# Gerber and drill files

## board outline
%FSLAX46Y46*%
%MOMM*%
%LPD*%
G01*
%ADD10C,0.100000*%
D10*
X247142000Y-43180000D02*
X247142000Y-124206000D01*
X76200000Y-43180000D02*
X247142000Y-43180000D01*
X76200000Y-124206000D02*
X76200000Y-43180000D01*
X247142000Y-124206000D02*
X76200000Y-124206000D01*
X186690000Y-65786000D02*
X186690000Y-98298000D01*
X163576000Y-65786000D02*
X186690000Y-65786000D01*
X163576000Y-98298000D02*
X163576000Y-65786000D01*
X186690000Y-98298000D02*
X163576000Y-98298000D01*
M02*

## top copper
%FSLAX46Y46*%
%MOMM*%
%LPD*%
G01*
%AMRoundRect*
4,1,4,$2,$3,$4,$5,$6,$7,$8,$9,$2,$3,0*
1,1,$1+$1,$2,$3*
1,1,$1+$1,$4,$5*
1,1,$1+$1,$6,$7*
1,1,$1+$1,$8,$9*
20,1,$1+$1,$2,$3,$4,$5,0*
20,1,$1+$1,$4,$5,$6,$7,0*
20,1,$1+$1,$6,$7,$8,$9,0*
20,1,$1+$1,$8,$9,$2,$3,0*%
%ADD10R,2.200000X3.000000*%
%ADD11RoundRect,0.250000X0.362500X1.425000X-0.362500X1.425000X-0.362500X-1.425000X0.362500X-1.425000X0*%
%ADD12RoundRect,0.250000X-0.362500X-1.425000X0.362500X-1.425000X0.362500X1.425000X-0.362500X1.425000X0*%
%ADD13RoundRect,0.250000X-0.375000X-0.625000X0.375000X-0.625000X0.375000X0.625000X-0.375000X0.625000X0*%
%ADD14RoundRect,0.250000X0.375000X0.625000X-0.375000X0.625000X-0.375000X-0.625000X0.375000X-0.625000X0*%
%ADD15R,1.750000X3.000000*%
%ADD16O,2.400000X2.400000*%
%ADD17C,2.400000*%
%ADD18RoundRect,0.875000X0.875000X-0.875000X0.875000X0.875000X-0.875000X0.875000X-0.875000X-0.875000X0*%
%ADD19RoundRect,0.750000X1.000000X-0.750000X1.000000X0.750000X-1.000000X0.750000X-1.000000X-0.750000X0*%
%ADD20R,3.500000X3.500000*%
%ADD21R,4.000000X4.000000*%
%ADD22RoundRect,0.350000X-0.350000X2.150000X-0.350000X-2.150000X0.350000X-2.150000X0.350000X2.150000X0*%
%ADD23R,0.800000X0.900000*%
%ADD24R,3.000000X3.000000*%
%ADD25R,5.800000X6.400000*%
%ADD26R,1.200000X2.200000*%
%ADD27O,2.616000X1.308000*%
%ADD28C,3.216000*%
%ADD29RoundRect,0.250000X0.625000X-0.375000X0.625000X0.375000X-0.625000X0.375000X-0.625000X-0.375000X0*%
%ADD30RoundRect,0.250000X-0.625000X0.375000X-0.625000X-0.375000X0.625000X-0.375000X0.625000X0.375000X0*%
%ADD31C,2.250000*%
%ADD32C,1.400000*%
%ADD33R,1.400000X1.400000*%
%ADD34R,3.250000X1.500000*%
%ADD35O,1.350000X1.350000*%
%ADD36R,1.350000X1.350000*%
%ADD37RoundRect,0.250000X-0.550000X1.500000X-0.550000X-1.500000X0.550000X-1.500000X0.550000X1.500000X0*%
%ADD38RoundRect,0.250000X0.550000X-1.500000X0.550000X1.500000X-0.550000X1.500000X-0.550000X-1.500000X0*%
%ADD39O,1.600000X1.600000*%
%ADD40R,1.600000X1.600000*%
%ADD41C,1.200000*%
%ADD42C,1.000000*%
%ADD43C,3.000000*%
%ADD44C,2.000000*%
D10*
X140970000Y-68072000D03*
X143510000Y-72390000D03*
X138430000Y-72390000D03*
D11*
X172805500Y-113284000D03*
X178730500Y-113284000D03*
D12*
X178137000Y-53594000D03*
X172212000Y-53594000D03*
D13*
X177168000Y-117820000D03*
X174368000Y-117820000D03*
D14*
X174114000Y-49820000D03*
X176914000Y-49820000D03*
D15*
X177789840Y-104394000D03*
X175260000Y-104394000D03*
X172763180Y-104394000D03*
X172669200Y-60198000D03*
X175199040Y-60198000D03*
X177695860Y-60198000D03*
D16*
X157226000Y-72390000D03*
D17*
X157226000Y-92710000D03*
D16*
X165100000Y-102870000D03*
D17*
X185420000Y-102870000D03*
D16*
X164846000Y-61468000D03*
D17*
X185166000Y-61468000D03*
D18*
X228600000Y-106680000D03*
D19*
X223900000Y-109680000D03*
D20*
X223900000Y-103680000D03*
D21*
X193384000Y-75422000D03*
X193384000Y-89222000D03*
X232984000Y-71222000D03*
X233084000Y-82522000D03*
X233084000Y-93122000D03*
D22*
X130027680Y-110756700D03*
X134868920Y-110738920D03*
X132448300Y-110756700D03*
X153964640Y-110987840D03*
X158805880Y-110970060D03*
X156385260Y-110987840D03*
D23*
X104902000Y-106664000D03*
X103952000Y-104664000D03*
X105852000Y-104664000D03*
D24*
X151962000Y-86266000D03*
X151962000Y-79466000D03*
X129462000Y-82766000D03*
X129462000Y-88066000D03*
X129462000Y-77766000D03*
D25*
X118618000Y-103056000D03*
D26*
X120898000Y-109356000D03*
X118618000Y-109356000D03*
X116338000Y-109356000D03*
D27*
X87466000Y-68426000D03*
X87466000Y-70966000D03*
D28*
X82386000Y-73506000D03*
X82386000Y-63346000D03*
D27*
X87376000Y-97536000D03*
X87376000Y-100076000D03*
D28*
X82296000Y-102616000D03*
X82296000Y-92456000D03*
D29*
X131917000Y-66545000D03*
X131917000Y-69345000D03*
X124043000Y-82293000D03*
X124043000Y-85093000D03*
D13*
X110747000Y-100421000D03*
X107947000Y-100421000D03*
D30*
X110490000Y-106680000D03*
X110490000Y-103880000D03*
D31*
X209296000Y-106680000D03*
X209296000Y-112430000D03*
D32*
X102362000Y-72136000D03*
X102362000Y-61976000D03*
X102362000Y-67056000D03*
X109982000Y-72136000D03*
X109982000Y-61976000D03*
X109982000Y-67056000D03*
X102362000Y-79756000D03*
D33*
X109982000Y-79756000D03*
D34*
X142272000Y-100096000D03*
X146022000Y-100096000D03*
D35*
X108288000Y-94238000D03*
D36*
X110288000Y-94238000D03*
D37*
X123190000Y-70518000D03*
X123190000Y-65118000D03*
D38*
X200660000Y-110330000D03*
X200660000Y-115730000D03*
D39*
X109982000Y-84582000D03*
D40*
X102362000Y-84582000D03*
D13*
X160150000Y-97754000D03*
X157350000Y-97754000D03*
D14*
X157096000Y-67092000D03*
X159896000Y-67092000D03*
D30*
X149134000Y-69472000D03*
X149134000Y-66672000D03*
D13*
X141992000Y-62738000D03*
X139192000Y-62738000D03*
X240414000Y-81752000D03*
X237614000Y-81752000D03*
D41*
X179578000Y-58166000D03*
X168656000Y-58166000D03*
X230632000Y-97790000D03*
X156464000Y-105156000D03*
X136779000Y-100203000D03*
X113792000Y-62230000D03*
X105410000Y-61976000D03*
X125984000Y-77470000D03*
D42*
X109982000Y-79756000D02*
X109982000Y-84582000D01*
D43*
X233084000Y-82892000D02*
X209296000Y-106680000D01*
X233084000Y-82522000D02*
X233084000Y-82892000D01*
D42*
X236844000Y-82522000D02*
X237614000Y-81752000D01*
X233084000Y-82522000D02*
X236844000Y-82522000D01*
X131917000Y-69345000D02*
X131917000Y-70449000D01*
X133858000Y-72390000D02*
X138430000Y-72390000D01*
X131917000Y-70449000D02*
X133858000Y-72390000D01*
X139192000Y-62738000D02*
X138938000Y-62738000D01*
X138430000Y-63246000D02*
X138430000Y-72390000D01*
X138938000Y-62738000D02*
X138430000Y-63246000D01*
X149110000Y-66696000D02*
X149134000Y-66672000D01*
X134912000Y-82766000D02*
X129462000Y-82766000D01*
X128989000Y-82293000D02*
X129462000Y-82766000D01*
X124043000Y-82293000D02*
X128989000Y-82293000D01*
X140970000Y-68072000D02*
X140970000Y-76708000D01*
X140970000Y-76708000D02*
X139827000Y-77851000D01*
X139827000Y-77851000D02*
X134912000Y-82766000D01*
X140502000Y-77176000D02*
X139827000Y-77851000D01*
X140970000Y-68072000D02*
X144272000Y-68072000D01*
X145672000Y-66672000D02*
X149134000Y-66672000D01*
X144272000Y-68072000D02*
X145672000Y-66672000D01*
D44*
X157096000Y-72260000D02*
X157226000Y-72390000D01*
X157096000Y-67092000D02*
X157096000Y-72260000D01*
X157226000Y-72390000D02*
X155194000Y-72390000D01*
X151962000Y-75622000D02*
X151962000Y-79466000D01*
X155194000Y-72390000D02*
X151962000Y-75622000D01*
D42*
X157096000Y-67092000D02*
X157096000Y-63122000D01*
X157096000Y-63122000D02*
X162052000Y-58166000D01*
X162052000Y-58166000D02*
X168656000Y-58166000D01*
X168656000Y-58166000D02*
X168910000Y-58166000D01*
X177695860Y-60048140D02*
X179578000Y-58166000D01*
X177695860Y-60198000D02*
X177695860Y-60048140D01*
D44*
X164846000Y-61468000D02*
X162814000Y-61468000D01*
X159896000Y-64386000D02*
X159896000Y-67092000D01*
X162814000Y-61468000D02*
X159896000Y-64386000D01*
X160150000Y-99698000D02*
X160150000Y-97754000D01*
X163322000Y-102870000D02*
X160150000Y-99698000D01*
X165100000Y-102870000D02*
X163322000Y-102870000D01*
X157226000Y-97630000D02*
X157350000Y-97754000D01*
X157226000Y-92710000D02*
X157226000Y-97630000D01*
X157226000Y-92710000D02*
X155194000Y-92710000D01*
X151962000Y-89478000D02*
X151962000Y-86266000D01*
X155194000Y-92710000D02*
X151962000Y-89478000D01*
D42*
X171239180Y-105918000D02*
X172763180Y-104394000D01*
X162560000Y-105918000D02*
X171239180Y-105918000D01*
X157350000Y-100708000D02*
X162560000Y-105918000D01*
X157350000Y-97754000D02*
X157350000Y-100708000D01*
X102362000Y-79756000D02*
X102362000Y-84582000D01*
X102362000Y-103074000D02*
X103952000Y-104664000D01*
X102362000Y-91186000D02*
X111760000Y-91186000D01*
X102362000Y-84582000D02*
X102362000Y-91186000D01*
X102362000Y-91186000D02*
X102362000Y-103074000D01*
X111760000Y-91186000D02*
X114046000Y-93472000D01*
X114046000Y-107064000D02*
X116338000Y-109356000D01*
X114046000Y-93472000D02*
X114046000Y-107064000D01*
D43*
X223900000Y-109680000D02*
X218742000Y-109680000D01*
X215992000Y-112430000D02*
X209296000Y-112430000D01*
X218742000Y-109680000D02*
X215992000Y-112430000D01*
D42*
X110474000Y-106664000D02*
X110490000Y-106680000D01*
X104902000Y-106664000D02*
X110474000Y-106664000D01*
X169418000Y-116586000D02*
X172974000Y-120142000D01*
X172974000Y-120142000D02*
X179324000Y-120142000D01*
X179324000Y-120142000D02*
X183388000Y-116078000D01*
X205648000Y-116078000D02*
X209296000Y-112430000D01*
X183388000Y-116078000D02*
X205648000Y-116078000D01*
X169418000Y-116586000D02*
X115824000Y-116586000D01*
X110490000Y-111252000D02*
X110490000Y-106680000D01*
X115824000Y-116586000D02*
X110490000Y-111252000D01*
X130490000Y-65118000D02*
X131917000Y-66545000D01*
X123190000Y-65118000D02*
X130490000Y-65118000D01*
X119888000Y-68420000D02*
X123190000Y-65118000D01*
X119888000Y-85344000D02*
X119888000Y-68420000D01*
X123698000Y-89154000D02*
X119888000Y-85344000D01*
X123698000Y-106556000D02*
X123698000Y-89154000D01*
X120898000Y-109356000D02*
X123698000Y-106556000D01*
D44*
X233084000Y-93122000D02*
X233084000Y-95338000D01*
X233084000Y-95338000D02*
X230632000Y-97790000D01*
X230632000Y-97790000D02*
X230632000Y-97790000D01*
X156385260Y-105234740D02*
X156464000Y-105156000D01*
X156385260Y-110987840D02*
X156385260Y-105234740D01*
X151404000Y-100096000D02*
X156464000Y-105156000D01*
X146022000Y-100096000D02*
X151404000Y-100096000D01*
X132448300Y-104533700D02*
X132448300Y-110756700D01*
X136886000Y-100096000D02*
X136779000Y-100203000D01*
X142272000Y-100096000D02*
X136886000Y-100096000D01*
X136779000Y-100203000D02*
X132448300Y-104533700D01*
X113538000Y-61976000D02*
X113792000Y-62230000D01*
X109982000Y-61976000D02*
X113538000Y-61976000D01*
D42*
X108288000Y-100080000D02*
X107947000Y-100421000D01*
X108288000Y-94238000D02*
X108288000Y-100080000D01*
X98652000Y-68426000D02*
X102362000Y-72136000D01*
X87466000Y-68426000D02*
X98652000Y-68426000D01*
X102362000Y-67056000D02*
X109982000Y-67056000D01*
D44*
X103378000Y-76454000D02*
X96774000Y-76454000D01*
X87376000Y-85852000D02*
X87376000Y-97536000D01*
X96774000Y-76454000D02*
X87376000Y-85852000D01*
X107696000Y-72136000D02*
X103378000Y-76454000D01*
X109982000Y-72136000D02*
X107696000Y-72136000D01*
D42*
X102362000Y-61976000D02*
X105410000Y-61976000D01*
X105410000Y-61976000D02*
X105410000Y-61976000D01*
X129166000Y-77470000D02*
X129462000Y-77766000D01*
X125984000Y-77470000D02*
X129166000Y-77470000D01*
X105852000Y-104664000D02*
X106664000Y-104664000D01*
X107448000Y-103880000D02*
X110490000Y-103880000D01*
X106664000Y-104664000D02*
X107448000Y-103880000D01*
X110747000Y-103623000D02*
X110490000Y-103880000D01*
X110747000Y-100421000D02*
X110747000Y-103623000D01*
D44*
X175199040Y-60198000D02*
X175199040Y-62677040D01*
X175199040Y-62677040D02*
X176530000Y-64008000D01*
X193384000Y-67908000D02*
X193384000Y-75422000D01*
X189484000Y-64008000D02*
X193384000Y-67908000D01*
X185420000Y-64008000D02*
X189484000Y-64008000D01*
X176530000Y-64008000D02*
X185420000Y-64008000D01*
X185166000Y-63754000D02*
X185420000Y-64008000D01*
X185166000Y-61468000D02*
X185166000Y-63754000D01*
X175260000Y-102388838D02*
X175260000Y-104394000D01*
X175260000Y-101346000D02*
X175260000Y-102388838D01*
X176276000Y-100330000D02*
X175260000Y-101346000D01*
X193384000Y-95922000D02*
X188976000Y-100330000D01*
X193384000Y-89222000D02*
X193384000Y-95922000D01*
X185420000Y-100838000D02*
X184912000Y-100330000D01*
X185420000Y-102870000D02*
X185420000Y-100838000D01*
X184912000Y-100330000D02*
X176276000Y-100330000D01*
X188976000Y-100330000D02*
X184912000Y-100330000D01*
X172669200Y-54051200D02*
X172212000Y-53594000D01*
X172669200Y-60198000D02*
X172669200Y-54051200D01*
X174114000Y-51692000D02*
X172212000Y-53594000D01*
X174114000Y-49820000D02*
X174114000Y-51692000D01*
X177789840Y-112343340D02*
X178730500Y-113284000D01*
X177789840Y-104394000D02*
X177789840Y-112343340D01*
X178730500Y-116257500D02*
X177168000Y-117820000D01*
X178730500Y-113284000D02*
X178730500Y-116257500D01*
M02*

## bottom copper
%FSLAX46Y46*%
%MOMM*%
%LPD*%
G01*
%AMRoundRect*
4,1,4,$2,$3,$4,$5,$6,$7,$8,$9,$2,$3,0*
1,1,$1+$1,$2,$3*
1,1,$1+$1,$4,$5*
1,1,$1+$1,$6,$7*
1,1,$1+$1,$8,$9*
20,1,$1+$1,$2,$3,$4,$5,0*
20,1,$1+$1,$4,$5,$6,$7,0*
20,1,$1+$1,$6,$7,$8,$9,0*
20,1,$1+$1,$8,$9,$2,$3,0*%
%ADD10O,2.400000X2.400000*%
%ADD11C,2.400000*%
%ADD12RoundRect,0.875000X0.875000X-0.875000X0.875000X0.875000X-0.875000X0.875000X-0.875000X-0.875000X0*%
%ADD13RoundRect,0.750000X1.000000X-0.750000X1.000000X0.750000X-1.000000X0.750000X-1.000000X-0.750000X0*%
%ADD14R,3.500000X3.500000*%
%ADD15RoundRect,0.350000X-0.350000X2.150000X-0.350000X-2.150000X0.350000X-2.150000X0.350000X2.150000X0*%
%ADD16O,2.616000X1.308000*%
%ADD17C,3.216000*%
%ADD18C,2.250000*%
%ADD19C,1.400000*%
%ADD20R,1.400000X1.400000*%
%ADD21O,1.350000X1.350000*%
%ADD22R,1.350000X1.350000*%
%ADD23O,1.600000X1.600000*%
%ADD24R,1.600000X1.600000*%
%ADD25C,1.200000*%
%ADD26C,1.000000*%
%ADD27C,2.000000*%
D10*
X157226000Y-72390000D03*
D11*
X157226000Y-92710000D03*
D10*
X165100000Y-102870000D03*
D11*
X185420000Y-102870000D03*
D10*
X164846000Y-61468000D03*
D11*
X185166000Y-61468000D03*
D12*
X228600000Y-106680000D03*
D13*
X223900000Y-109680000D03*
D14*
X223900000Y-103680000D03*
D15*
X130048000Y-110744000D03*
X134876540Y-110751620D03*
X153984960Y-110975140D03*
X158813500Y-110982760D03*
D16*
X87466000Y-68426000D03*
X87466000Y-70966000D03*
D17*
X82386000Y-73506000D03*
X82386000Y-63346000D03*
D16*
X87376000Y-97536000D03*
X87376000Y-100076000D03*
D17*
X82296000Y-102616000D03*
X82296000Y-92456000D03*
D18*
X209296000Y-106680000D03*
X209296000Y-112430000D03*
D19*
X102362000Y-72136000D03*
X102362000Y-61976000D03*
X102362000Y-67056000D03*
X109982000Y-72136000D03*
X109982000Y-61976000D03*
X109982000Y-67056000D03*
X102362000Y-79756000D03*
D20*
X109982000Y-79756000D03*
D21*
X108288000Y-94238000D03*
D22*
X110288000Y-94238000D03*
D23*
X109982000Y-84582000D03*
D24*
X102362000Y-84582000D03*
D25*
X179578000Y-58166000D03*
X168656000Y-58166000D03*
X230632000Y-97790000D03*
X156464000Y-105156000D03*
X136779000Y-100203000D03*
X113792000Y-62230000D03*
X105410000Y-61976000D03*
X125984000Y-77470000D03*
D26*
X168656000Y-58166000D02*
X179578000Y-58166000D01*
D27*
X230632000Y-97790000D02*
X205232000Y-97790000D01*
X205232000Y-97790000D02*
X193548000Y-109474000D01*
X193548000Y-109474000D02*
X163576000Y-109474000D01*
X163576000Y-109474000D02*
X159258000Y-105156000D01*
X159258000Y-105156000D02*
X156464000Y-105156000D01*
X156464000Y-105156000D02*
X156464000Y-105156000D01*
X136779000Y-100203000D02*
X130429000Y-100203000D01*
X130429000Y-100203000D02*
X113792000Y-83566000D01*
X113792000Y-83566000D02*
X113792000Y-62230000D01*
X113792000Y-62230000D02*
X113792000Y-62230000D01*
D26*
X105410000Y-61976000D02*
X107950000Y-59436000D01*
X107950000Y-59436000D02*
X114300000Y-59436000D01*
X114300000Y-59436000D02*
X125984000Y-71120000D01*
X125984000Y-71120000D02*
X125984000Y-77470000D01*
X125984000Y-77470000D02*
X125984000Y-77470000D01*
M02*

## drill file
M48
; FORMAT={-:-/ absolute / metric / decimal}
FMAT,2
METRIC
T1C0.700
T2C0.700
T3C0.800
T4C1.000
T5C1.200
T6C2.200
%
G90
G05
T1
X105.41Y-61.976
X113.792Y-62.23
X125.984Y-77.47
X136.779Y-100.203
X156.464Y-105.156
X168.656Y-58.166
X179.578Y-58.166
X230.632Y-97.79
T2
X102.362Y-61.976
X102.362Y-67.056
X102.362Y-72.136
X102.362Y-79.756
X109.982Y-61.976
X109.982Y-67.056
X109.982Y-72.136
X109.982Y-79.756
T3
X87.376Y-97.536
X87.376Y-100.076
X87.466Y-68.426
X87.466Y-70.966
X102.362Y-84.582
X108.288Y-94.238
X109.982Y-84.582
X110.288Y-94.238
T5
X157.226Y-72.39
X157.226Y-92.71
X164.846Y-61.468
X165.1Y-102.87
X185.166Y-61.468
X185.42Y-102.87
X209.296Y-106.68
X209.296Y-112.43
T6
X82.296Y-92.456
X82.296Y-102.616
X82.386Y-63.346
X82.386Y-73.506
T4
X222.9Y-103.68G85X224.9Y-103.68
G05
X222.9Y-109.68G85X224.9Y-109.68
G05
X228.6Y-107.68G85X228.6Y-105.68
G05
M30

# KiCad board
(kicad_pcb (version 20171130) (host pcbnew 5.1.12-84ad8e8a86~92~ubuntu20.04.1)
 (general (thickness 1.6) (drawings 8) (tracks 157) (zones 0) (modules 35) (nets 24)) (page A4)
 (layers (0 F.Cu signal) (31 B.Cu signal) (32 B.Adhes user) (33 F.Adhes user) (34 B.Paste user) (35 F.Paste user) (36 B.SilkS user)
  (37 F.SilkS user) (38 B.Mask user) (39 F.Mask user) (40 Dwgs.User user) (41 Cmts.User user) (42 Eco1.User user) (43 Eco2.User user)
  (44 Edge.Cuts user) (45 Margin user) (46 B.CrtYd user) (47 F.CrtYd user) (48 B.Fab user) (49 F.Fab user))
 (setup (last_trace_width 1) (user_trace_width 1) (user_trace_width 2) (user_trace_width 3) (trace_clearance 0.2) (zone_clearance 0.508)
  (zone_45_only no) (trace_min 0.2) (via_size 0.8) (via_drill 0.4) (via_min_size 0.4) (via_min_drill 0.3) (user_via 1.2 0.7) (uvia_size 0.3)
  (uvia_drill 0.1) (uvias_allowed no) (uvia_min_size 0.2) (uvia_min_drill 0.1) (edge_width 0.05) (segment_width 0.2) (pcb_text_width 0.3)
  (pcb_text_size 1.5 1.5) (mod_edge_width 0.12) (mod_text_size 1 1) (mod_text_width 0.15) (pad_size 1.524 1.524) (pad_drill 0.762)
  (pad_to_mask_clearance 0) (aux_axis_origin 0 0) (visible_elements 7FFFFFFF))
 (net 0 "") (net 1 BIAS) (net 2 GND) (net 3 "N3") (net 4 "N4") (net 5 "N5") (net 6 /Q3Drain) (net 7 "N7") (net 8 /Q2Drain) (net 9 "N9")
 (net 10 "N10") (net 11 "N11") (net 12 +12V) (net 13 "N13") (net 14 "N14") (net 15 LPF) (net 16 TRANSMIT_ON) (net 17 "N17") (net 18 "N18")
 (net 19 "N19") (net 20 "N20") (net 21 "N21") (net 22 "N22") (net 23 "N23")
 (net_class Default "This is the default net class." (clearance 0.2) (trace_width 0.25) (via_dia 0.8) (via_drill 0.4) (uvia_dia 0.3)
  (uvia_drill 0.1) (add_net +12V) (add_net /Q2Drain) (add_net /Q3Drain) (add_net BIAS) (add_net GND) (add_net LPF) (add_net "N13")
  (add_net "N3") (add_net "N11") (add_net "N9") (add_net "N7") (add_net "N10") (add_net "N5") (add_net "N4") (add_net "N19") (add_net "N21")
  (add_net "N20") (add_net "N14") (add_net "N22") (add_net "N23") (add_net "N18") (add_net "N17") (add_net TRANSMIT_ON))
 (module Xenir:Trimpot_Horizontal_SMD (layer F.Cu) (at 135.636 70.358 90)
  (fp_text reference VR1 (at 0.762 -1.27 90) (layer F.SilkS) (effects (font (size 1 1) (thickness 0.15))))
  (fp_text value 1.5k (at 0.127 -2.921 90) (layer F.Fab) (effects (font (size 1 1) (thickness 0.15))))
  (pad 2 smd rect (at 2.286 5.334 90) (size 3 2.2) (layers F.Cu F.Paste F.Mask) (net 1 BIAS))
  (pad 3 smd rect (at -2.032 7.874 90) (size 3 2.2) (layers F.Cu F.Paste F.Mask) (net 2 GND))
  (pad 1 smd rect (at -2.032 2.794 90) (size 3 2.2) (layers F.Cu F.Paste F.Mask) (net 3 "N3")))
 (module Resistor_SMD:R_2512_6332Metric (layer F.Cu) (at 175.768 113.284 180)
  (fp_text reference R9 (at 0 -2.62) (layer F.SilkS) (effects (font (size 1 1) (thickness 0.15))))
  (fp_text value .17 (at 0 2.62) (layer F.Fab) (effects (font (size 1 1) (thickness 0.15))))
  (pad 2 smd roundrect (at 2.9625 0 180) (size 1.225 3.35) (layers F.Cu F.Paste F.Mask) (roundrect_rratio 0.204082) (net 2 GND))
  (pad 1 smd roundrect (at -2.9625 0 180) (size 1.225 3.35) (layers F.Cu F.Paste F.Mask) (roundrect_rratio 0.204082) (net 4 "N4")))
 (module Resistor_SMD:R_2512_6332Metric (layer F.Cu) (at 175.1745 53.594)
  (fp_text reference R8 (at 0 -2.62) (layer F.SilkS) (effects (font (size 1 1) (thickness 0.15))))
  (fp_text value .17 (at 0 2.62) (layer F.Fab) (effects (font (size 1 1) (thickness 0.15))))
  (pad 2 smd roundrect (at 2.9625 0) (size 1.225 3.35) (layers F.Cu F.Paste F.Mask) (roundrect_rratio 0.204082) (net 2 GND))
  (pad 1 smd roundrect (at -2.9625 0) (size 1.225 3.35) (layers F.Cu F.Paste F.Mask) (roundrect_rratio 0.204082) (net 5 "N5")))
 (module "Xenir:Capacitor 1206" (layer F.Cu) (at 175.768 115.57)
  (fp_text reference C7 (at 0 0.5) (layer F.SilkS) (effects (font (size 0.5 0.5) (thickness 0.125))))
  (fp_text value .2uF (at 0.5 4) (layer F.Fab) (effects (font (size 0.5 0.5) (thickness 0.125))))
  (pad 2 smd roundrect (at 1.4 2.25) (size 1.25 1.75) (layers F.Cu F.Paste F.Mask) (roundrect_rratio 0.2) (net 4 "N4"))
  (pad 1 smd roundrect (at -1.4 2.25) (size 1.25 1.75) (layers F.Cu F.Paste F.Mask) (roundrect_rratio 0.2) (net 2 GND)))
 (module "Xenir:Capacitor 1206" (layer F.Cu) (at 175.514 52.07 180)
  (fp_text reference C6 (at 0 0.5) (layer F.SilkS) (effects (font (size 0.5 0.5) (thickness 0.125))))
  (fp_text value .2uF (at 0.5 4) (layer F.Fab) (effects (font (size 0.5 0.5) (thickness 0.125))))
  (pad 2 smd roundrect (at 1.4 2.25 180) (size 1.25 1.75) (layers F.Cu F.Paste F.Mask) (roundrect_rratio 0.2) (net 5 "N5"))
  (pad 1 smd roundrect (at -1.4 2.25 180) (size 1.25 1.75) (layers F.Cu F.Paste F.Mask) (roundrect_rratio 0.2) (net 2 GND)))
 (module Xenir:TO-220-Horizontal (layer F.Cu) (at 175.45304 98.43918)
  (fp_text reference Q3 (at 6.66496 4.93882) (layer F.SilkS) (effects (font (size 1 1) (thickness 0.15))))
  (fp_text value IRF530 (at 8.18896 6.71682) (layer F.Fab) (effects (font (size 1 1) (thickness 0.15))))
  (pad 3 smd rect (at 2.3368 5.95482) (size 1.75 3) (layers F.Cu F.Paste F.Mask) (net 4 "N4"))
  (pad 2 smd rect (at -0.19304 5.95482) (size 1.75 3) (layers F.Cu F.Paste F.Mask) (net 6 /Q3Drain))
  (pad 1 smd rect (at -2.68986 5.95482) (size 1.75 3) (layers F.Cu F.Paste F.Mask) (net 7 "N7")))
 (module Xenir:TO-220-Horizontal (layer F.Cu) (at 175.006 66.15282 180)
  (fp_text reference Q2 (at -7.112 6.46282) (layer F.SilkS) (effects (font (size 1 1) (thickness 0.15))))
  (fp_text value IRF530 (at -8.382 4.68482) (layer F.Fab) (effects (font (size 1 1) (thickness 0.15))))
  (pad 3 smd rect (at 2.3368 5.95482 180) (size 1.75 3) (layers F.Cu F.Paste F.Mask) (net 5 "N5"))
  (pad 2 smd rect (at -0.19304 5.95482 180) (size 1.75 3) (layers F.Cu F.Paste F.Mask) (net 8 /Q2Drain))
  (pad 1 smd rect (at -2.68986 5.95482 180) (size 1.75 3) (layers F.Cu F.Paste F.Mask) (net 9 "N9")))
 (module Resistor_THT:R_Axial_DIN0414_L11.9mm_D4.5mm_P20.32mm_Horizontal (layer F.Cu) (at 157.226 92.71 90)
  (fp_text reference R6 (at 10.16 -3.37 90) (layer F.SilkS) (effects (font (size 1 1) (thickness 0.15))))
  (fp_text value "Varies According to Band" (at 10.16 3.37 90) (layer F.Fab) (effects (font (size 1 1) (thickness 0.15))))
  (pad 2 thru_hole oval (at 20.32 0 90) (size 2.4 2.4) (drill 1.2) (layers *.Cu *.Mask) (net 9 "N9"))
  (pad 1 thru_hole circle (at 0 0 90) (size 2.4 2.4) (drill 1.2) (layers *.Cu *.Mask) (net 7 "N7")))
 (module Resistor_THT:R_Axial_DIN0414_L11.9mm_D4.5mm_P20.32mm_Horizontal (layer F.Cu) (at 185.42 102.87 180)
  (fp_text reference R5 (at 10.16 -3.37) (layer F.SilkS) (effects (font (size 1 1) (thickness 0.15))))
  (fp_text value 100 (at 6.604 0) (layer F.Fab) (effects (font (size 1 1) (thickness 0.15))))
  (pad 2 thru_hole oval (at 20.32 0 180) (size 2.4 2.4) (drill 1.2) (layers *.Cu *.Mask) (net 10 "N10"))
  (pad 1 thru_hole circle (at 0 0 180) (size 2.4 2.4) (drill 1.2) (layers *.Cu *.Mask) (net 6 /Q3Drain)))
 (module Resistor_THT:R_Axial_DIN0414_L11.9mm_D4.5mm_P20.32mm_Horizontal (layer F.Cu) (at 185.166 61.468 180)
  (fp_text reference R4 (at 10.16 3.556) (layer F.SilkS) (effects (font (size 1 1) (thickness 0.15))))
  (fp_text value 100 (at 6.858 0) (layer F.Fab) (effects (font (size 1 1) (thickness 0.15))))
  (pad 2 thru_hole oval (at 20.32 0 180) (size 2.4 2.4) (drill 1.2) (layers *.Cu *.Mask) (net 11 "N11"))
  (pad 1 thru_hole circle (at 0 0 180) (size 2.4 2.4) (drill 1.2) (layers *.Cu *.Mask) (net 8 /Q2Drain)))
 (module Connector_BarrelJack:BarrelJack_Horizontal (layer F.Cu) (at 223.9 103.68 90)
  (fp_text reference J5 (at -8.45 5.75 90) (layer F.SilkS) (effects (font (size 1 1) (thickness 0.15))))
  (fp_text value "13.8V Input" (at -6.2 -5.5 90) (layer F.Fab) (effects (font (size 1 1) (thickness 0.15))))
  (pad 3 thru_hole roundrect (at -3 4.7 90) (size 3.5 3.5) (drill oval 3 1) (layers *.Cu *.Mask) (roundrect_rratio 0.25))
  (pad 2 thru_hole roundrect (at -6 0 90) (size 3 3.5) (drill oval 1 3) (layers *.Cu *.Mask) (roundrect_rratio 0.25) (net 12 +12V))
  (pad 1 thru_hole rect (at 0 0 90) (size 3.5 3.5) (drill oval 1 3) (layers *.Cu *.Mask) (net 2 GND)))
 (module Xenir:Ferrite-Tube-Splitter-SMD (layer F.Cu) (at 214.884 99.822 180)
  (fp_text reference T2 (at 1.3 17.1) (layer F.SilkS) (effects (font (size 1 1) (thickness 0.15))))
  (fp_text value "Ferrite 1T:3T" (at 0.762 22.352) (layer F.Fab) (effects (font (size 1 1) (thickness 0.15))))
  (pad 5 smd rect (at 21.5 24.4 180) (size 4 4) (layers F.Cu F.Paste F.Mask) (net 8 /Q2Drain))
  (pad 3 smd rect (at 21.5 10.6 180) (size 4 4) (layers F.Cu F.Paste F.Mask) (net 6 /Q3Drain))
  (pad 2 smd rect (at -18.1 28.6 180) (size 4 4) (layers F.Cu F.Paste F.Mask) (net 2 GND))
  (pad 4 smd rect (at -18.2 17.3 180) (size 4 4) (layers F.Cu F.Paste F.Mask) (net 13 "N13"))
  (pad 1 smd rect (at -18.2 6.7 180) (size 4 4) (layers F.Cu F.Paste F.Mask) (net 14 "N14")))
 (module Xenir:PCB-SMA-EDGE (layer F.Cu) (at 137.60704 110.76686 270)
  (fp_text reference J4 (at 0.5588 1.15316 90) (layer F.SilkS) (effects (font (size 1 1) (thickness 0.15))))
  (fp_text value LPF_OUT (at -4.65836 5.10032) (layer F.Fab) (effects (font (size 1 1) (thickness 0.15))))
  (pad 2 smd roundrect (at -0.02286 7.55904 270) (size 5 1.4) (layers B.Cu F.Paste F.Mask) (roundrect_rratio 0.25) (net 2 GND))
  (pad 2 smd roundrect (at -0.01524 2.7305 270) (size 5 1.4) (layers B.Cu F.Paste F.Mask) (roundrect_rratio 0.25) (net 2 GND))
  (pad 2 smd roundrect (at -0.01016 7.57936 270) (size 5 1.4) (layers F.Cu F.Paste F.Mask) (roundrect_rratio 0.25) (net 2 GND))
  (pad 2 smd roundrect (at -0.02794 2.73812 270) (size 5 1.4) (layers F.Cu F.Paste F.Mask) (roundrect_rratio 0.25) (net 2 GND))
  (pad 1 smd roundrect (at -0.01016 5.15874 270) (size 5 1.4) (layers F.Cu F.Paste F.Mask) (roundrect_rratio 0.25) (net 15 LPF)))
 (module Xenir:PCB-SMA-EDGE (layer F.Cu) (at 161.544 110.998 270)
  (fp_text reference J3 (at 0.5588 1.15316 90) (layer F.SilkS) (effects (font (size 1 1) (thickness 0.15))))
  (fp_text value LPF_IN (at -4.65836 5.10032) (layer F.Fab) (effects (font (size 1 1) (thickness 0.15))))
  (pad 2 smd roundrect (at -0.02286 7.55904 270) (size 5 1.4) (layers B.Cu F.Paste F.Mask) (roundrect_rratio 0.25) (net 2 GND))
  (pad 2 smd roundrect (at -0.01524 2.7305 270) (size 5 1.4) (layers B.Cu F.Paste F.Mask) (roundrect_rratio 0.25) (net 2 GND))
  (pad 2 smd roundrect (at -0.01016 7.57936 270) (size 5 1.4) (layers F.Cu F.Paste F.Mask) (roundrect_rratio 0.25) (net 2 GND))
  (pad 2 smd roundrect (at -0.02794 2.73812 270) (size 5 1.4) (layers F.Cu F.Paste F.Mask) (roundrect_rratio 0.25) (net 2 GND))
  (pad 1 smd roundrect (at -0.01016 5.15874 270) (size 5 1.4) (layers F.Cu F.Paste F.Mask) (roundrect_rratio 0.25) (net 14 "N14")))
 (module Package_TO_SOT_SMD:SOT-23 (layer F.Cu) (at 104.902 105.664 270)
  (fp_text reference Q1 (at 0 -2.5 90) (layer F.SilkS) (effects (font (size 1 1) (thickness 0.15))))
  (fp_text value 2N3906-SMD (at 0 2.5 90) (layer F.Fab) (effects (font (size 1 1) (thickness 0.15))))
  (pad 3 smd rect (at 1 0 270) (size 0.9 0.8) (layers F.Cu F.Paste F.Mask) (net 12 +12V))
  (pad 2 smd rect (at -1 0.95 270) (size 0.9 0.8) (layers F.Cu F.Paste F.Mask) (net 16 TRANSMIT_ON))
  (pad 1 smd rect (at -1 -0.95 270) (size 0.9 0.8) (layers F.Cu F.Paste F.Mask) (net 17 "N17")))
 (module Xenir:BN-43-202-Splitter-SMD (layer F.Cu) (at 140.462 70.866)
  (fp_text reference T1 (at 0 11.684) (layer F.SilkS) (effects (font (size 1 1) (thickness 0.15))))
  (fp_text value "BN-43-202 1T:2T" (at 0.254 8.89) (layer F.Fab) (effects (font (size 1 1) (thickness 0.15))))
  (pad 5 smd rect (at 11.5 15.4) (size 3 3) (layers F.Cu F.Paste F.Mask) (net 7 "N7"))
  (pad 3 smd rect (at 11.5 8.6) (size 3 3) (layers F.Cu F.Paste F.Mask) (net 9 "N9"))
  (pad 4 smd rect (at -11 11.9) (size 3 3) (layers F.Cu F.Paste F.Mask) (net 1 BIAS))
  (pad 2 smd rect (at -11 17.2) (size 3 3) (layers F.Cu F.Paste F.Mask) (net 2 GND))
  (pad 1 smd rect (at -11 6.9) (size 3 3) (layers F.Cu F.Paste F.Mask) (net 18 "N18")))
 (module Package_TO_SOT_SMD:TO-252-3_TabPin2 (layer F.Cu) (at 118.618 105.156 90)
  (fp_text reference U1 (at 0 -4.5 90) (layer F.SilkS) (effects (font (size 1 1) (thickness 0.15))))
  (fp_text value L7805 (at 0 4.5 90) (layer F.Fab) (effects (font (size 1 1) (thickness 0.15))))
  (pad "" smd rect (at 0.425 1.525 90) (size 3.05 2.75) (layers F.Paste))
  (pad "" smd rect (at 3.775 -1.525 90) (size 3.05 2.75) (layers F.Paste))
  (pad "" smd rect (at 0.425 -1.525 90) (size 3.05 2.75) (layers F.Paste))
  (pad "" smd rect (at 3.775 1.525 90) (size 3.05 2.75) (layers F.Paste))
  (pad 2 smd rect (at 2.1 0 90) (size 6.4 5.8) (layers F.Cu F.Mask) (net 2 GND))
  (pad 3 smd rect (at -4.2 2.28 90) (size 2.2 1.2) (layers F.Cu F.Paste F.Mask) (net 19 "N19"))
  (pad 2 smd rect (at -4.2 0 90) (size 2.2 1.2) (layers F.Cu F.Paste F.Mask) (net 2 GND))
  (pad 1 smd rect (at -4.2 -2.28 90) (size 2.2 1.2) (layers F.Cu F.Paste F.Mask) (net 16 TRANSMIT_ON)))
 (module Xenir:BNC (layer F.Cu) (at 83.566 68.326 90)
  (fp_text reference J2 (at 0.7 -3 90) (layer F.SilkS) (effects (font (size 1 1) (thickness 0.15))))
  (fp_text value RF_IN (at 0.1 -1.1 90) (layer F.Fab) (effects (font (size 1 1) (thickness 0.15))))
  (pad S thru_hole oval (at -0.1 3.9 180) (size 2.616 1.308) (drill 0.8) (layers *.Cu *.Mask) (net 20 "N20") (solder_mask_margin 0.1016))
  (pad GND thru_hole oval (at -2.64 3.9 180) (size 2.616 1.308) (drill 0.8) (layers *.Cu *.Mask) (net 2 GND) (solder_mask_margin 0.1016))
  (pad 3 thru_hole circle (at -5.18 -1.18 90) (size 3.216 3.216) (drill 2.2) (layers *.Cu *.Mask) (solder_mask_margin 0.1016))
  (pad 4 thru_hole circle (at 4.98 -1.18 90) (size 3.216 3.216) (drill 2.2) (layers *.Cu *.Mask) (solder_mask_margin 0.1016)))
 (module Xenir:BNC (layer F.Cu) (at 83.476 97.436 90)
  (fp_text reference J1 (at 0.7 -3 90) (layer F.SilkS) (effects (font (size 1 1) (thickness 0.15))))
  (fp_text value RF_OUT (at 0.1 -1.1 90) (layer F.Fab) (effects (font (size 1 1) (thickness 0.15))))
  (pad S thru_hole oval (at -0.1 3.9 180) (size 2.616 1.308) (drill 0.8) (layers *.Cu *.Mask) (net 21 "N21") (solder_mask_margin 0.1016))
  (pad GND thru_hole oval (at -2.64 3.9 180) (size 2.616 1.308) (drill 0.8) (layers *.Cu *.Mask) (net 2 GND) (solder_mask_margin 0.1016))
  (pad 3 thru_hole circle (at -5.18 -1.18 90) (size 3.216 3.216) (drill 2.2) (layers *.Cu *.Mask) (solder_mask_margin 0.1016))
  (pad 4 thru_hole circle (at 4.98 -1.18 90) (size 3.216 3.216) (drill 2.2) (layers *.Cu *.Mask) (solder_mask_margin 0.1016)))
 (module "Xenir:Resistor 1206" (layer F.Cu) (at 129.54 67.818 90)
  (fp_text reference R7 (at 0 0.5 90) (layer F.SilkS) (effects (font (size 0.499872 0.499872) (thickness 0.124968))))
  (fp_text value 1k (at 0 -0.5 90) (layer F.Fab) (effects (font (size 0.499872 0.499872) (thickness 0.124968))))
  (pad 2 smd roundrect (at 1.273 2.377 90) (size 1.25 1.75) (layers F.Cu F.Paste F.Mask) (roundrect_rratio 0.2) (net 19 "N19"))
  (pad 1 smd roundrect (at -1.527 2.377 90) (size 1.25 1.75) (layers F.Cu F.Paste F.Mask) (roundrect_rratio 0.2) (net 3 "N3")))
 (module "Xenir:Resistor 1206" (layer F.Cu) (at 121.666 83.566 90)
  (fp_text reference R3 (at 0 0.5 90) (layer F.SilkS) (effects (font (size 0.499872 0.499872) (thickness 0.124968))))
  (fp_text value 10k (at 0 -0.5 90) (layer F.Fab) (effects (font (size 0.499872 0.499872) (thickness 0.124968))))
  (pad 2 smd roundrect (at 1.273 2.377 90) (size 1.25 1.75) (layers F.Cu F.Paste F.Mask) (roundrect_rratio 0.2) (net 1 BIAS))
  (pad 1 smd roundrect (at -1.527 2.377 90) (size 1.25 1.75) (layers F.Cu F.Paste F.Mask) (roundrect_rratio 0.2) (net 2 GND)))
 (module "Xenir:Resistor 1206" (layer F.Cu) (at 109.474 98.044)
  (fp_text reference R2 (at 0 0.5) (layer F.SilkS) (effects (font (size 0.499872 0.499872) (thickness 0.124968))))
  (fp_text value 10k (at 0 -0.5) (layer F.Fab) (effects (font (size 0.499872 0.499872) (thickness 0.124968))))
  (pad 2 smd roundrect (at 1.273 2.377) (size 1.25 1.75) (layers F.Cu F.Paste F.Mask) (roundrect_rratio 0.2) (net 17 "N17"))
  (pad 1 smd roundrect (at -1.527 2.377) (size 1.25 1.75) (layers F.Cu F.Paste F.Mask) (roundrect_rratio 0.2) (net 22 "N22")))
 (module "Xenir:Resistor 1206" (layer F.Cu) (at 112.867 105.407 270)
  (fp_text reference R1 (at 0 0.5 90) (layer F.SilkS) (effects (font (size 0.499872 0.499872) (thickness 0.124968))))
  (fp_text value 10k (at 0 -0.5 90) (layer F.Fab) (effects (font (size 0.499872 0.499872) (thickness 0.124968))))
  (pad 2 smd roundrect (at 1.273 2.377 270) (size 1.25 1.75) (layers F.Cu F.Paste F.Mask) (roundrect_rratio 0.2) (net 12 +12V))
  (pad 1 smd roundrect (at -1.527 2.377 270) (size 1.25 1.75) (layers F.Cu F.Paste F.Mask) (roundrect_rratio 0.2) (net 17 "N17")))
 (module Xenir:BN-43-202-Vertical (layer F.Cu) (at 209.296 117.43 180)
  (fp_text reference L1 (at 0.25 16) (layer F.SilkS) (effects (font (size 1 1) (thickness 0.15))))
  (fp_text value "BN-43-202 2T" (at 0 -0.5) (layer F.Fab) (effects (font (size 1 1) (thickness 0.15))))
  (pad 2 thru_hole circle (at 0 10.75 180) (size 2.25 2.25) (drill 1.2) (layers *.Cu *.Mask) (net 13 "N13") (solder_mask_margin 0.1016))
  (pad 1 thru_hole circle (at 0 5 180) (size 2.25 2.25) (drill 1.2) (layers *.Cu *.Mask) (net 12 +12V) (solder_mask_margin 0.1016)))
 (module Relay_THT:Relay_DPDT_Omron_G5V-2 (layer F.Cu) (at 109.982 79.756 180)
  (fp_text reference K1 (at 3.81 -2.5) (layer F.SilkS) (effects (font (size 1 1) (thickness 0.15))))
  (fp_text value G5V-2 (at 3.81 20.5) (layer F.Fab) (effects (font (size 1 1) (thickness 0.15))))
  (pad 13 thru_hole circle (at 7.62 7.62 180) (size 1.4 1.4) (drill 0.7) (layers *.Cu *.Mask) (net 20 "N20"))
  (pad 9 thru_hole circle (at 7.62 17.78 180) (size 1.4 1.4) (drill 0.7) (layers *.Cu *.Mask) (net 18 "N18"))
  (pad 11 thru_hole circle (at 7.62 12.7 180) (size 1.4 1.4) (drill 0.7) (layers *.Cu *.Mask) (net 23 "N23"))
  (pad 4 thru_hole circle (at 0 7.62 180) (size 1.4 1.4) (drill 0.7) (layers *.Cu *.Mask) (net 21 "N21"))
  (pad 8 thru_hole circle (at 0 17.78 180) (size 1.4 1.4) (drill 0.7) (layers *.Cu *.Mask) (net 15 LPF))
  (pad 6 thru_hole circle (at 0 12.7 180) (size 1.4 1.4) (drill 0.7) (layers *.Cu *.Mask) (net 23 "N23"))
  (pad 16 thru_hole circle (at 7.62 0 180) (size 1.4 1.4) (drill 0.7) (layers *.Cu *.Mask) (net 16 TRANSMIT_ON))
  (pad 1 thru_hole rect (at 0 0 180) (size 1.4 1.4) (drill 0.7) (layers *.Cu *.Mask) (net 2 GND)))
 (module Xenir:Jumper (layer F.Cu) (at 144.272 101.346 180)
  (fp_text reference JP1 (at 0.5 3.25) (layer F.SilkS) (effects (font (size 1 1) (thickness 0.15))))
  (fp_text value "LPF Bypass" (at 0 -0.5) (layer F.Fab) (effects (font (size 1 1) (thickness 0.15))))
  (pad 2 smd rect (at 2 1.25 180) (size 3.25 1.5) (layers F.Cu F.Mask) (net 15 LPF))
  (pad 1 smd rect (at -1.75 1.25 180) (size 3.25 1.5) (layers F.Cu F.Mask) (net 14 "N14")))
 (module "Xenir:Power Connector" (layer F.Cu) (at 113.538 94.488 270)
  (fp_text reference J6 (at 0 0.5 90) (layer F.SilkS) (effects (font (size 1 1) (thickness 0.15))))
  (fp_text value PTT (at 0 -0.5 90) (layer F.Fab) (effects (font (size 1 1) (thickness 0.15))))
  (pad 2 thru_hole oval (at -0.25 5.25 270) (size 1.35 1.35) (drill 0.8) (layers *.Cu *.Mask) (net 22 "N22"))
  (pad 1 thru_hole rect (at -0.25 3.25 270) (size 1.35 1.35) (drill 0.8) (layers *.Cu *.Mask) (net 2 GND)))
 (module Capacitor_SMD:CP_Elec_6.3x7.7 (layer F.Cu) (at 123.19 67.818 270)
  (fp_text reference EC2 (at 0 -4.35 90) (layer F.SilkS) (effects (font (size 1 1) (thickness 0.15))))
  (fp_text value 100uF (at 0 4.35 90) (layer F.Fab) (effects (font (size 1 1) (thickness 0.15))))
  (pad 2 smd roundrect (at 2.7 0 270) (size 3.5 1.6) (layers F.Cu F.Paste F.Mask) (roundrect_rratio 0.15625) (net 2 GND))
  (pad 1 smd roundrect (at -2.7 0 270) (size 3.5 1.6) (layers F.Cu F.Paste F.Mask) (roundrect_rratio 0.15625) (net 19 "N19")))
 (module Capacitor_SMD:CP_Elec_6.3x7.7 (layer F.Cu) (at 200.66 113.03 90)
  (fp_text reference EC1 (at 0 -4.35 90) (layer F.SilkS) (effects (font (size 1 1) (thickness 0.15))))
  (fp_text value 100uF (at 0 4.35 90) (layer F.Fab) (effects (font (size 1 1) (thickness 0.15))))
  (pad 2 smd roundrect (at 2.7 0 90) (size 3.5 1.6) (layers F.Cu F.Paste F.Mask) (roundrect_rratio 0.15625) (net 2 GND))
  (pad 1 smd roundrect (at -2.7 0 90) (size 3.5 1.6) (layers F.Cu F.Paste F.Mask) (roundrect_rratio 0.15625) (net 12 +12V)))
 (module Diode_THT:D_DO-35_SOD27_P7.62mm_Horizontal (layer F.Cu) (at 102.362 84.582)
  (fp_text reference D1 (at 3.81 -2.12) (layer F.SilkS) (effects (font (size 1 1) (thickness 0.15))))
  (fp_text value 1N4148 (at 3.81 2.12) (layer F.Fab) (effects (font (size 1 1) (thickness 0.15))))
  (pad 2 thru_hole oval (at 7.62 0) (size 1.6 1.6) (drill 0.8) (layers *.Cu *.Mask) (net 2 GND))
  (pad 1 thru_hole rect (at 0 0) (size 1.6 1.6) (drill 0.8) (layers *.Cu *.Mask) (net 16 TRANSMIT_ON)))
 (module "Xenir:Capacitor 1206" (layer F.Cu) (at 158.75 95.504)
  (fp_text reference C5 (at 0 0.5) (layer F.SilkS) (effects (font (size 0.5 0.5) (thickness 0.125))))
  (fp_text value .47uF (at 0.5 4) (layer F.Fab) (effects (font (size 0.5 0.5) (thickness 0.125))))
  (pad 2 smd roundrect (at 1.4 2.25) (size 1.25 1.75) (layers F.Cu F.Paste F.Mask) (roundrect_rratio 0.2) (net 10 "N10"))
  (pad 1 smd roundrect (at -1.4 2.25) (size 1.25 1.75) (layers F.Cu F.Paste F.Mask) (roundrect_rratio 0.2) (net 7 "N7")))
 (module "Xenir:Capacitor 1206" (layer F.Cu) (at 158.496 69.342 180)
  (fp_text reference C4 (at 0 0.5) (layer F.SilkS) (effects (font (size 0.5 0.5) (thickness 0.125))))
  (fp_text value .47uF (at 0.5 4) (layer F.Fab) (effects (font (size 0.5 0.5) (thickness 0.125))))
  (pad 2 smd roundrect (at 1.4 2.25 180) (size 1.25 1.75) (layers F.Cu F.Paste F.Mask) (roundrect_rratio 0.2) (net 9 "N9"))
  (pad 1 smd roundrect (at -1.4 2.25 180) (size 1.25 1.75) (layers F.Cu F.Paste F.Mask) (roundrect_rratio 0.2) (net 11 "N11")))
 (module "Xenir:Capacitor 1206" (layer F.Cu) (at 151.384 68.072 270)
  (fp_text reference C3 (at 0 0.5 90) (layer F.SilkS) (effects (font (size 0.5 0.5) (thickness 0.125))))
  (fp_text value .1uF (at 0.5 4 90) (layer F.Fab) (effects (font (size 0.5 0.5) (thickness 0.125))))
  (pad 2 smd roundrect (at 1.4 2.25 270) (size 1.25 1.75) (layers F.Cu F.Paste F.Mask) (roundrect_rratio 0.2) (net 2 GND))
  (pad 1 smd roundrect (at -1.4 2.25 270) (size 1.25 1.75) (layers F.Cu F.Paste F.Mask) (roundrect_rratio 0.2) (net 1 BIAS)))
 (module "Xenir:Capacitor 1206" (layer F.Cu) (at 140.592 60.488)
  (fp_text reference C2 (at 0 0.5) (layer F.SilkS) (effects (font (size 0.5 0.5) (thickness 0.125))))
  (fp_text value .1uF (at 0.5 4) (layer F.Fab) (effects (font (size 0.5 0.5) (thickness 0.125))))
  (pad 2 smd roundrect (at 1.4 2.25) (size 1.25 1.75) (layers F.Cu F.Paste F.Mask) (roundrect_rratio 0.2) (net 2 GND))
  (pad 1 smd roundrect (at -1.4 2.25) (size 1.25 1.75) (layers F.Cu F.Paste F.Mask) (roundrect_rratio 0.2) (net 3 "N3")))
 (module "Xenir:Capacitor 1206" (layer F.Cu) (at 239.014 79.502)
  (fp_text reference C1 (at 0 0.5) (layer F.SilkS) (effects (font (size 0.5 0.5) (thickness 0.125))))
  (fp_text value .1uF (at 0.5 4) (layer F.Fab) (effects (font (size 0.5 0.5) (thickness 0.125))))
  (pad 2 smd roundrect (at 1.4 2.25) (size 1.25 1.75) (layers F.Cu F.Paste F.Mask) (roundrect_rratio 0.2) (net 2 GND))
  (pad 1 smd roundrect (at -1.4 2.25) (size 1.25 1.75) (layers F.Cu F.Paste F.Mask) (roundrect_rratio 0.2) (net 13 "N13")))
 (gr_line (start 247.142 43.18) (end 247.142 124.206) (layer Edge.Cuts) (width 0.1))
 (gr_line (start 76.2 43.18) (end 247.142 43.18) (layer Edge.Cuts) (width 0.1))
 (gr_line (start 76.2 124.206) (end 76.2 43.18) (layer Edge.Cuts) (width 0.1))
 (gr_line (start 247.142 124.206) (end 76.2 124.206) (layer Edge.Cuts) (width 0.1))
 (gr_line (start 186.69 65.786) (end 186.69 98.298) (layer Edge.Cuts) (width 0.1))
 (gr_line (start 163.576 65.786) (end 186.69 65.786) (layer Edge.Cuts) (width 0.1))
 (gr_line (start 163.576 98.298) (end 163.576 65.786) (layer Edge.Cuts) (width 0.1))
 (gr_line (start 186.69 98.298) (end 163.576 98.298) (layer Edge.Cuts) (width 0.1))
 (segment (start 109.982 79.756) (end 109.982 84.582) (width 1) (layer F.Cu) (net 2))
 (segment (start 233.084 82.892) (end 209.296 106.68) (width 3) (layer F.Cu) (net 13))
 (segment (start 233.084 82.522) (end 233.084 82.892) (width 3) (layer F.Cu) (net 13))
 (segment (start 236.844 82.522) (end 237.614 81.752) (width 1) (layer F.Cu) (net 13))
 (segment (start 233.084 82.522) (end 236.844 82.522) (width 1) (layer F.Cu) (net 13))
 (segment (start 131.917 69.345) (end 131.917 70.449) (width 1) (layer F.Cu) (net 3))
 (segment (start 133.858 72.39) (end 138.43 72.39) (width 1) (layer F.Cu) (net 3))
 (segment (start 131.917 70.449) (end 133.858 72.39) (width 1) (layer F.Cu) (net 3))
 (segment (start 139.192 62.738) (end 138.938 62.738) (width 1) (layer F.Cu) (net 3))
 (segment (start 138.43 63.246) (end 138.43 72.39) (width 1) (layer F.Cu) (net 3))
 (segment (start 138.938 62.738) (end 138.43 63.246) (width 1) (layer F.Cu) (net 3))
 (segment (start 149.11 66.696) (end 149.134 66.672) (width 1) (layer F.Cu) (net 1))
 (segment (start 134.912 82.766) (end 129.462 82.766) (width 1) (layer F.Cu) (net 1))
 (segment (start 128.989 82.293) (end 129.462 82.766) (width 1) (layer F.Cu) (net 1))
 (segment (start 124.043 82.293) (end 128.989 82.293) (width 1) (layer F.Cu) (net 1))
 (segment (start 140.97 68.072) (end 140.97 76.708) (width 1) (layer F.Cu) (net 1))
 (segment (start 140.97 76.708) (end 139.827 77.851) (width 1) (layer F.Cu) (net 1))
 (segment (start 139.827 77.851) (end 134.912 82.766) (width 1) (layer F.Cu) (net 1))
 (segment (start 140.502 77.176) (end 139.827 77.851) (width 1) (layer F.Cu) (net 1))
 (segment (start 140.97 68.072) (end 144.272 68.072) (width 1) (layer F.Cu) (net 1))
 (segment (start 145.672 66.672) (end 149.134 66.672) (width 1) (layer F.Cu) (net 1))
 (segment (start 144.272 68.072) (end 145.672 66.672) (width 1) (layer F.Cu) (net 1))
 (via (at 179.578 58.166) (size 1.2) (drill 0.7) (layers F.Cu B.Cu) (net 9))
 (segment (start 157.096 72.26) (end 157.226 72.39) (width 2) (layer F.Cu) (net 9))
 (segment (start 157.096 67.092) (end 157.096 72.26) (width 2) (layer F.Cu) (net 9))
 (segment (start 157.226 72.39) (end 155.194 72.39) (width 2) (layer F.Cu) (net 9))
 (segment (start 151.962 75.622) (end 151.962 79.466) (width 2) (layer F.Cu) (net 9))
 (segment (start 155.194 72.39) (end 151.962 75.622) (width 2) (layer F.Cu) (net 9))
 (segment (start 157.096 67.092) (end 157.096 63.122) (width 1) (layer F.Cu) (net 9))
 (segment (start 157.096 63.122) (end 162.052 58.166) (width 1) (layer F.Cu) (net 9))
 (segment (start 162.052 58.166) (end 168.656 58.166) (width 1) (layer F.Cu) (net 9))
 (segment (start 168.656 58.166) (end 168.91 58.166) (width 1) (layer F.Cu) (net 9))
 (via (at 168.656 58.166) (size 1.2) (drill 0.7) (layers F.Cu B.Cu) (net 9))
 (segment (start 177.69586 60.04814) (end 179.578 58.166) (width 1) (layer F.Cu) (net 9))
 (segment (start 177.69586 60.198) (end 177.69586 60.04814) (width 1) (layer F.Cu) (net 9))
 (segment (start 168.656 58.166) (end 179.578 58.166) (width 1) (layer B.Cu) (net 9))
 (segment (start 164.846 61.468) (end 162.814 61.468) (width 2) (layer F.Cu) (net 11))
 (segment (start 159.896 64.386) (end 159.896 67.092) (width 2) (layer F.Cu) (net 11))
 (segment (start 162.814 61.468) (end 159.896 64.386) (width 2) (layer F.Cu) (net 11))
 (segment (start 160.15 99.698) (end 160.15 97.754) (width 2) (layer F.Cu) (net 10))
 (segment (start 163.322 102.87) (end 160.15 99.698) (width 2) (layer F.Cu) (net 10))
 (segment (start 165.1 102.87) (end 163.322 102.87) (width 2) (layer F.Cu) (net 10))
 (segment (start 157.226 97.63) (end 157.35 97.754) (width 2) (layer F.Cu) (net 7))
 (segment (start 157.226 92.71) (end 157.226 97.63) (width 2) (layer F.Cu) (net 7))
 (segment (start 157.226 92.71) (end 155.194 92.71) (width 2) (layer F.Cu) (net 7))
 (segment (start 151.962 89.478) (end 151.962 86.266) (width 2) (layer F.Cu) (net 7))
 (segment (start 155.194 92.71) (end 151.962 89.478) (width 2) (layer F.Cu) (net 7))
 (segment (start 171.23918 105.918) (end 172.76318 104.394) (width 1) (layer F.Cu) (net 7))
 (segment (start 162.56 105.918) (end 171.23918 105.918) (width 1) (layer F.Cu) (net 7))
 (segment (start 157.35 100.708) (end 162.56 105.918) (width 1) (layer F.Cu) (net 7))
 (segment (start 157.35 97.754) (end 157.35 100.708) (width 1) (layer F.Cu) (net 7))
 (segment (start 102.362 79.756) (end 102.362 84.582) (width 1) (layer F.Cu) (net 16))
 (segment (start 102.362 103.074) (end 103.952 104.664) (width 1) (layer F.Cu) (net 16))
 (segment (start 102.362 91.186) (end 111.76 91.186) (width 1) (layer F.Cu) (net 16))
 (segment (start 102.362 84.582) (end 102.362 91.186) (width 1) (layer F.Cu) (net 16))
 (segment (start 102.362 91.186) (end 102.362 103.074) (width 1) (layer F.Cu) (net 16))
 (segment (start 111.76 91.186) (end 114.046 93.472) (width 1) (layer F.Cu) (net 16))
 (segment (start 114.046 107.064) (end 116.338 109.356) (width 1) (layer F.Cu) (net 16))
 (segment (start 114.046 93.472) (end 114.046 107.064) (width 1) (layer F.Cu) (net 16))
 (segment (start 223.9 109.68) (end 218.742 109.68) (width 3) (layer F.Cu) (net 12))
 (segment (start 215.992 112.43) (end 209.296 112.43) (width 3) (layer F.Cu) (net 12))
 (segment (start 218.742 109.68) (end 215.992 112.43) (width 3) (layer F.Cu) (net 12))
 (segment (start 110.474 106.664) (end 110.49 106.68) (width 1) (layer F.Cu) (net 12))
 (segment (start 104.902 106.664) (end 110.474 106.664) (width 1) (layer F.Cu) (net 12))
 (segment (start 169.418 116.586) (end 172.974 120.142) (width 1) (layer F.Cu) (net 12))
 (segment (start 172.974 120.142) (end 179.324 120.142) (width 1) (layer F.Cu) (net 12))
 (segment (start 179.324 120.142) (end 183.388 116.078) (width 1) (layer F.Cu) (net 12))
 (segment (start 205.648 116.078) (end 209.296 112.43) (width 1) (layer F.Cu) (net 12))
 (segment (start 183.388 116.078) (end 205.648 116.078) (width 1) (layer F.Cu) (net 12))
 (segment (start 169.418 116.586) (end 115.824 116.586) (width 1) (layer F.Cu) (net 12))
 (segment (start 110.49 111.252) (end 110.49 106.68) (width 1) (layer F.Cu) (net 12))
 (segment (start 115.824 116.586) (end 110.49 111.252) (width 1) (layer F.Cu) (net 12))
 (segment (start 130.49 65.118) (end 131.917 66.545) (width 1) (layer F.Cu) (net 19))
 (segment (start 123.19 65.118) (end 130.49 65.118) (width 1) (layer F.Cu) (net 19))
 (segment (start 119.888 68.42) (end 123.19 65.118) (width 1) (layer F.Cu) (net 19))
 (segment (start 119.888 85.344) (end 119.888 68.42) (width 1) (layer F.Cu) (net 19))
 (segment (start 123.698 89.154) (end 119.888 85.344) (width 1) (layer F.Cu) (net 19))
 (segment (start 123.698 106.556) (end 123.698 89.154) (width 1) (layer F.Cu) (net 19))
 (segment (start 120.898 109.356) (end 123.698 106.556) (width 1) (layer F.Cu) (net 19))
 (segment (start 233.084 93.122) (end 233.084 95.338) (width 2) (layer F.Cu) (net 14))
 (segment (start 233.084 95.338) (end 230.632 97.79) (width 2) (layer F.Cu) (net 14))
 (segment (start 230.632 97.79) (end 230.632 97.79) (width 2) (layer F.Cu) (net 14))
 (via (at 230.632 97.79) (size 1.2) (drill 0.7) (layers F.Cu B.Cu) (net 14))
 (segment (start 230.632 97.79) (end 205.232 97.79) (width 2) (layer B.Cu) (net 14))
 (segment (start 205.232 97.79) (end 193.548 109.474) (width 2) (layer B.Cu) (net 14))
 (segment (start 193.548 109.474) (end 163.576 109.474) (width 2) (layer B.Cu) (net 14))
 (segment (start 163.576 109.474) (end 159.258 105.156) (width 2) (layer B.Cu) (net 14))
 (segment (start 159.258 105.156) (end 156.464 105.156) (width 2) (layer B.Cu) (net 14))
 (segment (start 156.464 105.156) (end 156.464 105.156) (width 2) (layer B.Cu) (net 14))
 (via (at 156.464 105.156) (size 1.2) (drill 0.7) (layers F.Cu B.Cu) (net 14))
 (segment (start 156.38526 105.23474) (end 156.464 105.156) (width 2) (layer F.Cu) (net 14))
 (segment (start 156.38526 110.98784) (end 156.38526 105.23474) (width 2) (layer F.Cu) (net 14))
 (segment (start 151.404 100.096) (end 156.464 105.156) (width 2) (layer F.Cu) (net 14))
 (segment (start 146.022 100.096) (end 151.404 100.096) (width 2) (layer F.Cu) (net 14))
 (segment (start 132.4483 104.5337) (end 132.4483 110.7567) (width 2) (layer F.Cu) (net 15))
 (segment (start 136.886 100.096) (end 136.779 100.203) (width 2) (layer F.Cu) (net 15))
 (segment (start 142.272 100.096) (end 136.886 100.096) (width 2) (layer F.Cu) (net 15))
 (segment (start 136.779 100.203) (end 132.4483 104.5337) (width 2) (layer F.Cu) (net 15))
 (via (at 136.779 100.203) (size 1.2) (drill 0.7) (layers F.Cu B.Cu) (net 15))
 (segment (start 136.779 100.203) (end 130.429 100.203) (width 2) (layer B.Cu) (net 15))
 (segment (start 130.429 100.203) (end 113.792 83.566) (width 2) (layer B.Cu) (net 15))
 (segment (start 113.792 83.566) (end 113.792 62.23) (width 2) (layer B.Cu) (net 15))
 (segment (start 113.792 62.23) (end 113.792 62.23) (width 2) (layer B.Cu) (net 15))
 (via (at 113.792 62.23) (size 1.2) (drill 0.7) (layers F.Cu B.Cu) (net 15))
 (segment (start 113.538 61.976) (end 113.792 62.23) (width 2) (layer F.Cu) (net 15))
 (segment (start 109.982 61.976) (end 113.538 61.976) (width 2) (layer F.Cu) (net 15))
 (segment (start 108.288 100.08) (end 107.947 100.421) (width 1) (layer F.Cu) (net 22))
 (segment (start 108.288 94.238) (end 108.288 100.08) (width 1) (layer F.Cu) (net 22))
 (segment (start 98.652 68.426) (end 102.362 72.136) (width 1) (layer F.Cu) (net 20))
 (segment (start 87.466 68.426) (end 98.652 68.426) (width 1) (layer F.Cu) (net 20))
 (segment (start 102.362 67.056) (end 109.982 67.056) (width 1) (layer F.Cu) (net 23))
 (segment (start 103.378 76.454) (end 96.774 76.454) (width 2) (layer F.Cu) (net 21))
 (segment (start 87.376 85.852) (end 87.376 97.536) (width 2) (layer F.Cu) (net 21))
 (segment (start 96.774 76.454) (end 87.376 85.852) (width 2) (layer F.Cu) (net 21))
 (segment (start 107.696 72.136) (end 103.378 76.454) (width 2) (layer F.Cu) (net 21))
 (segment (start 109.982 72.136) (end 107.696 72.136) (width 2) (layer F.Cu) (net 21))
 (segment (start 102.362 61.976) (end 105.41 61.976) (width 1) (layer F.Cu) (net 18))
 (segment (start 105.41 61.976) (end 105.41 61.976) (width 1) (layer F.Cu) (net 18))
 (via (at 105.41 61.976) (size 1.2) (drill 0.7) (layers F.Cu B.Cu) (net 18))
 (segment (start 105.41 61.976) (end 107.95 59.436) (width 1) (layer B.Cu) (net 18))
 (segment (start 107.95 59.436) (end 114.3 59.436) (width 1) (layer B.Cu) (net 18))
 (segment (start 114.3 59.436) (end 125.984 71.12) (width 1) (layer B.Cu) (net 18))
 (segment (start 125.984 71.12) (end 125.984 77.47) (width 1) (layer B.Cu) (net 18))
 (segment (start 125.984 77.47) (end 125.984 77.47) (width 1) (layer B.Cu) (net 18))
 (via (at 125.984 77.47) (size 1.2) (drill 0.7) (layers F.Cu B.Cu) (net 18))
 (segment (start 129.166 77.47) (end 129.462 77.766) (width 1) (layer F.Cu) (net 18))
 (segment (start 125.984 77.47) (end 129.166 77.47) (width 1) (layer F.Cu) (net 18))
 (segment (start 105.852 104.664) (end 106.664 104.664) (width 1) (layer F.Cu) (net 17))
 (segment (start 107.448 103.88) (end 110.49 103.88) (width 1) (layer F.Cu) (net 17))
 (segment (start 106.664 104.664) (end 107.448 103.88) (width 1) (layer F.Cu) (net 17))
 (segment (start 110.747 103.623) (end 110.49 103.88) (width 1) (layer F.Cu) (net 17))
 (segment (start 110.747 100.421) (end 110.747 103.623) (width 1) (layer F.Cu) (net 17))
 (segment (start 175.19904 60.198) (end 175.19904 62.67704) (width 2) (layer F.Cu) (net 8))
 (segment (start 175.19904 62.67704) (end 176.53 64.008) (width 2) (layer F.Cu) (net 8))
 (segment (start 193.384 67.908) (end 193.384 75.422) (width 2) (layer F.Cu) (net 8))
 (segment (start 189.484 64.008) (end 193.384 67.908) (width 2) (layer F.Cu) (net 8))
 (segment (start 185.42 64.008) (end 189.484 64.008) (width 2) (layer F.Cu) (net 8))
 (segment (start 176.53 64.008) (end 185.42 64.008) (width 2) (layer F.Cu) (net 8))
 (segment (start 185.166 63.754) (end 185.42 64.008) (width 2) (layer F.Cu) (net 8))
 (segment (start 185.166 61.468) (end 185.166 63.754) (width 2) (layer F.Cu) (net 8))
 (segment (start 175.26 102.388838) (end 175.26 104.394) (width 2) (layer F.Cu) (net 6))
 (segment (start 175.26 101.346) (end 175.26 102.388838) (width 2) (layer F.Cu) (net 6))
 (segment (start 176.276 100.33) (end 175.26 101.346) (width 2) (layer F.Cu) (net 6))
 (segment (start 193.384 95.922) (end 188.976 100.33) (width 2) (layer F.Cu) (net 6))
 (segment (start 193.384 89.222) (end 193.384 95.922) (width 2) (layer F.Cu) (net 6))
 (segment (start 185.42 100.838) (end 184.912 100.33) (width 2) (layer F.Cu) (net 6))
 (segment (start 185.42 102.87) (end 185.42 100.838) (width 2) (layer F.Cu) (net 6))
 (segment (start 184.912 100.33) (end 176.276 100.33) (width 2) (layer F.Cu) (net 6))
 (segment (start 188.976 100.33) (end 184.912 100.33) (width 2) (layer F.Cu) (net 6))
 (segment (start 172.6692 54.0512) (end 172.212 53.594) (width 2) (layer F.Cu) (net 5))
 (segment (start 172.6692 60.198) (end 172.6692 54.0512) (width 2) (layer F.Cu) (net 5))
 (segment (start 174.114 51.692) (end 172.212 53.594) (width 2) (layer F.Cu) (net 5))
 (segment (start 174.114 49.82) (end 174.114 51.692) (width 2) (layer F.Cu) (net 5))
 (segment (start 177.78984 112.34334) (end 178.7305 113.284) (width 2) (layer F.Cu) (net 4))
 (segment (start 177.78984 104.394) (end 177.78984 112.34334) (width 2) (layer F.Cu) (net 4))
 (segment (start 178.7305 116.2575) (end 177.168 117.82) (width 2) (layer F.Cu) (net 4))
 (segment (start 178.7305 113.284) (end 178.7305 116.2575) (width 2) (layer F.Cu) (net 4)))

